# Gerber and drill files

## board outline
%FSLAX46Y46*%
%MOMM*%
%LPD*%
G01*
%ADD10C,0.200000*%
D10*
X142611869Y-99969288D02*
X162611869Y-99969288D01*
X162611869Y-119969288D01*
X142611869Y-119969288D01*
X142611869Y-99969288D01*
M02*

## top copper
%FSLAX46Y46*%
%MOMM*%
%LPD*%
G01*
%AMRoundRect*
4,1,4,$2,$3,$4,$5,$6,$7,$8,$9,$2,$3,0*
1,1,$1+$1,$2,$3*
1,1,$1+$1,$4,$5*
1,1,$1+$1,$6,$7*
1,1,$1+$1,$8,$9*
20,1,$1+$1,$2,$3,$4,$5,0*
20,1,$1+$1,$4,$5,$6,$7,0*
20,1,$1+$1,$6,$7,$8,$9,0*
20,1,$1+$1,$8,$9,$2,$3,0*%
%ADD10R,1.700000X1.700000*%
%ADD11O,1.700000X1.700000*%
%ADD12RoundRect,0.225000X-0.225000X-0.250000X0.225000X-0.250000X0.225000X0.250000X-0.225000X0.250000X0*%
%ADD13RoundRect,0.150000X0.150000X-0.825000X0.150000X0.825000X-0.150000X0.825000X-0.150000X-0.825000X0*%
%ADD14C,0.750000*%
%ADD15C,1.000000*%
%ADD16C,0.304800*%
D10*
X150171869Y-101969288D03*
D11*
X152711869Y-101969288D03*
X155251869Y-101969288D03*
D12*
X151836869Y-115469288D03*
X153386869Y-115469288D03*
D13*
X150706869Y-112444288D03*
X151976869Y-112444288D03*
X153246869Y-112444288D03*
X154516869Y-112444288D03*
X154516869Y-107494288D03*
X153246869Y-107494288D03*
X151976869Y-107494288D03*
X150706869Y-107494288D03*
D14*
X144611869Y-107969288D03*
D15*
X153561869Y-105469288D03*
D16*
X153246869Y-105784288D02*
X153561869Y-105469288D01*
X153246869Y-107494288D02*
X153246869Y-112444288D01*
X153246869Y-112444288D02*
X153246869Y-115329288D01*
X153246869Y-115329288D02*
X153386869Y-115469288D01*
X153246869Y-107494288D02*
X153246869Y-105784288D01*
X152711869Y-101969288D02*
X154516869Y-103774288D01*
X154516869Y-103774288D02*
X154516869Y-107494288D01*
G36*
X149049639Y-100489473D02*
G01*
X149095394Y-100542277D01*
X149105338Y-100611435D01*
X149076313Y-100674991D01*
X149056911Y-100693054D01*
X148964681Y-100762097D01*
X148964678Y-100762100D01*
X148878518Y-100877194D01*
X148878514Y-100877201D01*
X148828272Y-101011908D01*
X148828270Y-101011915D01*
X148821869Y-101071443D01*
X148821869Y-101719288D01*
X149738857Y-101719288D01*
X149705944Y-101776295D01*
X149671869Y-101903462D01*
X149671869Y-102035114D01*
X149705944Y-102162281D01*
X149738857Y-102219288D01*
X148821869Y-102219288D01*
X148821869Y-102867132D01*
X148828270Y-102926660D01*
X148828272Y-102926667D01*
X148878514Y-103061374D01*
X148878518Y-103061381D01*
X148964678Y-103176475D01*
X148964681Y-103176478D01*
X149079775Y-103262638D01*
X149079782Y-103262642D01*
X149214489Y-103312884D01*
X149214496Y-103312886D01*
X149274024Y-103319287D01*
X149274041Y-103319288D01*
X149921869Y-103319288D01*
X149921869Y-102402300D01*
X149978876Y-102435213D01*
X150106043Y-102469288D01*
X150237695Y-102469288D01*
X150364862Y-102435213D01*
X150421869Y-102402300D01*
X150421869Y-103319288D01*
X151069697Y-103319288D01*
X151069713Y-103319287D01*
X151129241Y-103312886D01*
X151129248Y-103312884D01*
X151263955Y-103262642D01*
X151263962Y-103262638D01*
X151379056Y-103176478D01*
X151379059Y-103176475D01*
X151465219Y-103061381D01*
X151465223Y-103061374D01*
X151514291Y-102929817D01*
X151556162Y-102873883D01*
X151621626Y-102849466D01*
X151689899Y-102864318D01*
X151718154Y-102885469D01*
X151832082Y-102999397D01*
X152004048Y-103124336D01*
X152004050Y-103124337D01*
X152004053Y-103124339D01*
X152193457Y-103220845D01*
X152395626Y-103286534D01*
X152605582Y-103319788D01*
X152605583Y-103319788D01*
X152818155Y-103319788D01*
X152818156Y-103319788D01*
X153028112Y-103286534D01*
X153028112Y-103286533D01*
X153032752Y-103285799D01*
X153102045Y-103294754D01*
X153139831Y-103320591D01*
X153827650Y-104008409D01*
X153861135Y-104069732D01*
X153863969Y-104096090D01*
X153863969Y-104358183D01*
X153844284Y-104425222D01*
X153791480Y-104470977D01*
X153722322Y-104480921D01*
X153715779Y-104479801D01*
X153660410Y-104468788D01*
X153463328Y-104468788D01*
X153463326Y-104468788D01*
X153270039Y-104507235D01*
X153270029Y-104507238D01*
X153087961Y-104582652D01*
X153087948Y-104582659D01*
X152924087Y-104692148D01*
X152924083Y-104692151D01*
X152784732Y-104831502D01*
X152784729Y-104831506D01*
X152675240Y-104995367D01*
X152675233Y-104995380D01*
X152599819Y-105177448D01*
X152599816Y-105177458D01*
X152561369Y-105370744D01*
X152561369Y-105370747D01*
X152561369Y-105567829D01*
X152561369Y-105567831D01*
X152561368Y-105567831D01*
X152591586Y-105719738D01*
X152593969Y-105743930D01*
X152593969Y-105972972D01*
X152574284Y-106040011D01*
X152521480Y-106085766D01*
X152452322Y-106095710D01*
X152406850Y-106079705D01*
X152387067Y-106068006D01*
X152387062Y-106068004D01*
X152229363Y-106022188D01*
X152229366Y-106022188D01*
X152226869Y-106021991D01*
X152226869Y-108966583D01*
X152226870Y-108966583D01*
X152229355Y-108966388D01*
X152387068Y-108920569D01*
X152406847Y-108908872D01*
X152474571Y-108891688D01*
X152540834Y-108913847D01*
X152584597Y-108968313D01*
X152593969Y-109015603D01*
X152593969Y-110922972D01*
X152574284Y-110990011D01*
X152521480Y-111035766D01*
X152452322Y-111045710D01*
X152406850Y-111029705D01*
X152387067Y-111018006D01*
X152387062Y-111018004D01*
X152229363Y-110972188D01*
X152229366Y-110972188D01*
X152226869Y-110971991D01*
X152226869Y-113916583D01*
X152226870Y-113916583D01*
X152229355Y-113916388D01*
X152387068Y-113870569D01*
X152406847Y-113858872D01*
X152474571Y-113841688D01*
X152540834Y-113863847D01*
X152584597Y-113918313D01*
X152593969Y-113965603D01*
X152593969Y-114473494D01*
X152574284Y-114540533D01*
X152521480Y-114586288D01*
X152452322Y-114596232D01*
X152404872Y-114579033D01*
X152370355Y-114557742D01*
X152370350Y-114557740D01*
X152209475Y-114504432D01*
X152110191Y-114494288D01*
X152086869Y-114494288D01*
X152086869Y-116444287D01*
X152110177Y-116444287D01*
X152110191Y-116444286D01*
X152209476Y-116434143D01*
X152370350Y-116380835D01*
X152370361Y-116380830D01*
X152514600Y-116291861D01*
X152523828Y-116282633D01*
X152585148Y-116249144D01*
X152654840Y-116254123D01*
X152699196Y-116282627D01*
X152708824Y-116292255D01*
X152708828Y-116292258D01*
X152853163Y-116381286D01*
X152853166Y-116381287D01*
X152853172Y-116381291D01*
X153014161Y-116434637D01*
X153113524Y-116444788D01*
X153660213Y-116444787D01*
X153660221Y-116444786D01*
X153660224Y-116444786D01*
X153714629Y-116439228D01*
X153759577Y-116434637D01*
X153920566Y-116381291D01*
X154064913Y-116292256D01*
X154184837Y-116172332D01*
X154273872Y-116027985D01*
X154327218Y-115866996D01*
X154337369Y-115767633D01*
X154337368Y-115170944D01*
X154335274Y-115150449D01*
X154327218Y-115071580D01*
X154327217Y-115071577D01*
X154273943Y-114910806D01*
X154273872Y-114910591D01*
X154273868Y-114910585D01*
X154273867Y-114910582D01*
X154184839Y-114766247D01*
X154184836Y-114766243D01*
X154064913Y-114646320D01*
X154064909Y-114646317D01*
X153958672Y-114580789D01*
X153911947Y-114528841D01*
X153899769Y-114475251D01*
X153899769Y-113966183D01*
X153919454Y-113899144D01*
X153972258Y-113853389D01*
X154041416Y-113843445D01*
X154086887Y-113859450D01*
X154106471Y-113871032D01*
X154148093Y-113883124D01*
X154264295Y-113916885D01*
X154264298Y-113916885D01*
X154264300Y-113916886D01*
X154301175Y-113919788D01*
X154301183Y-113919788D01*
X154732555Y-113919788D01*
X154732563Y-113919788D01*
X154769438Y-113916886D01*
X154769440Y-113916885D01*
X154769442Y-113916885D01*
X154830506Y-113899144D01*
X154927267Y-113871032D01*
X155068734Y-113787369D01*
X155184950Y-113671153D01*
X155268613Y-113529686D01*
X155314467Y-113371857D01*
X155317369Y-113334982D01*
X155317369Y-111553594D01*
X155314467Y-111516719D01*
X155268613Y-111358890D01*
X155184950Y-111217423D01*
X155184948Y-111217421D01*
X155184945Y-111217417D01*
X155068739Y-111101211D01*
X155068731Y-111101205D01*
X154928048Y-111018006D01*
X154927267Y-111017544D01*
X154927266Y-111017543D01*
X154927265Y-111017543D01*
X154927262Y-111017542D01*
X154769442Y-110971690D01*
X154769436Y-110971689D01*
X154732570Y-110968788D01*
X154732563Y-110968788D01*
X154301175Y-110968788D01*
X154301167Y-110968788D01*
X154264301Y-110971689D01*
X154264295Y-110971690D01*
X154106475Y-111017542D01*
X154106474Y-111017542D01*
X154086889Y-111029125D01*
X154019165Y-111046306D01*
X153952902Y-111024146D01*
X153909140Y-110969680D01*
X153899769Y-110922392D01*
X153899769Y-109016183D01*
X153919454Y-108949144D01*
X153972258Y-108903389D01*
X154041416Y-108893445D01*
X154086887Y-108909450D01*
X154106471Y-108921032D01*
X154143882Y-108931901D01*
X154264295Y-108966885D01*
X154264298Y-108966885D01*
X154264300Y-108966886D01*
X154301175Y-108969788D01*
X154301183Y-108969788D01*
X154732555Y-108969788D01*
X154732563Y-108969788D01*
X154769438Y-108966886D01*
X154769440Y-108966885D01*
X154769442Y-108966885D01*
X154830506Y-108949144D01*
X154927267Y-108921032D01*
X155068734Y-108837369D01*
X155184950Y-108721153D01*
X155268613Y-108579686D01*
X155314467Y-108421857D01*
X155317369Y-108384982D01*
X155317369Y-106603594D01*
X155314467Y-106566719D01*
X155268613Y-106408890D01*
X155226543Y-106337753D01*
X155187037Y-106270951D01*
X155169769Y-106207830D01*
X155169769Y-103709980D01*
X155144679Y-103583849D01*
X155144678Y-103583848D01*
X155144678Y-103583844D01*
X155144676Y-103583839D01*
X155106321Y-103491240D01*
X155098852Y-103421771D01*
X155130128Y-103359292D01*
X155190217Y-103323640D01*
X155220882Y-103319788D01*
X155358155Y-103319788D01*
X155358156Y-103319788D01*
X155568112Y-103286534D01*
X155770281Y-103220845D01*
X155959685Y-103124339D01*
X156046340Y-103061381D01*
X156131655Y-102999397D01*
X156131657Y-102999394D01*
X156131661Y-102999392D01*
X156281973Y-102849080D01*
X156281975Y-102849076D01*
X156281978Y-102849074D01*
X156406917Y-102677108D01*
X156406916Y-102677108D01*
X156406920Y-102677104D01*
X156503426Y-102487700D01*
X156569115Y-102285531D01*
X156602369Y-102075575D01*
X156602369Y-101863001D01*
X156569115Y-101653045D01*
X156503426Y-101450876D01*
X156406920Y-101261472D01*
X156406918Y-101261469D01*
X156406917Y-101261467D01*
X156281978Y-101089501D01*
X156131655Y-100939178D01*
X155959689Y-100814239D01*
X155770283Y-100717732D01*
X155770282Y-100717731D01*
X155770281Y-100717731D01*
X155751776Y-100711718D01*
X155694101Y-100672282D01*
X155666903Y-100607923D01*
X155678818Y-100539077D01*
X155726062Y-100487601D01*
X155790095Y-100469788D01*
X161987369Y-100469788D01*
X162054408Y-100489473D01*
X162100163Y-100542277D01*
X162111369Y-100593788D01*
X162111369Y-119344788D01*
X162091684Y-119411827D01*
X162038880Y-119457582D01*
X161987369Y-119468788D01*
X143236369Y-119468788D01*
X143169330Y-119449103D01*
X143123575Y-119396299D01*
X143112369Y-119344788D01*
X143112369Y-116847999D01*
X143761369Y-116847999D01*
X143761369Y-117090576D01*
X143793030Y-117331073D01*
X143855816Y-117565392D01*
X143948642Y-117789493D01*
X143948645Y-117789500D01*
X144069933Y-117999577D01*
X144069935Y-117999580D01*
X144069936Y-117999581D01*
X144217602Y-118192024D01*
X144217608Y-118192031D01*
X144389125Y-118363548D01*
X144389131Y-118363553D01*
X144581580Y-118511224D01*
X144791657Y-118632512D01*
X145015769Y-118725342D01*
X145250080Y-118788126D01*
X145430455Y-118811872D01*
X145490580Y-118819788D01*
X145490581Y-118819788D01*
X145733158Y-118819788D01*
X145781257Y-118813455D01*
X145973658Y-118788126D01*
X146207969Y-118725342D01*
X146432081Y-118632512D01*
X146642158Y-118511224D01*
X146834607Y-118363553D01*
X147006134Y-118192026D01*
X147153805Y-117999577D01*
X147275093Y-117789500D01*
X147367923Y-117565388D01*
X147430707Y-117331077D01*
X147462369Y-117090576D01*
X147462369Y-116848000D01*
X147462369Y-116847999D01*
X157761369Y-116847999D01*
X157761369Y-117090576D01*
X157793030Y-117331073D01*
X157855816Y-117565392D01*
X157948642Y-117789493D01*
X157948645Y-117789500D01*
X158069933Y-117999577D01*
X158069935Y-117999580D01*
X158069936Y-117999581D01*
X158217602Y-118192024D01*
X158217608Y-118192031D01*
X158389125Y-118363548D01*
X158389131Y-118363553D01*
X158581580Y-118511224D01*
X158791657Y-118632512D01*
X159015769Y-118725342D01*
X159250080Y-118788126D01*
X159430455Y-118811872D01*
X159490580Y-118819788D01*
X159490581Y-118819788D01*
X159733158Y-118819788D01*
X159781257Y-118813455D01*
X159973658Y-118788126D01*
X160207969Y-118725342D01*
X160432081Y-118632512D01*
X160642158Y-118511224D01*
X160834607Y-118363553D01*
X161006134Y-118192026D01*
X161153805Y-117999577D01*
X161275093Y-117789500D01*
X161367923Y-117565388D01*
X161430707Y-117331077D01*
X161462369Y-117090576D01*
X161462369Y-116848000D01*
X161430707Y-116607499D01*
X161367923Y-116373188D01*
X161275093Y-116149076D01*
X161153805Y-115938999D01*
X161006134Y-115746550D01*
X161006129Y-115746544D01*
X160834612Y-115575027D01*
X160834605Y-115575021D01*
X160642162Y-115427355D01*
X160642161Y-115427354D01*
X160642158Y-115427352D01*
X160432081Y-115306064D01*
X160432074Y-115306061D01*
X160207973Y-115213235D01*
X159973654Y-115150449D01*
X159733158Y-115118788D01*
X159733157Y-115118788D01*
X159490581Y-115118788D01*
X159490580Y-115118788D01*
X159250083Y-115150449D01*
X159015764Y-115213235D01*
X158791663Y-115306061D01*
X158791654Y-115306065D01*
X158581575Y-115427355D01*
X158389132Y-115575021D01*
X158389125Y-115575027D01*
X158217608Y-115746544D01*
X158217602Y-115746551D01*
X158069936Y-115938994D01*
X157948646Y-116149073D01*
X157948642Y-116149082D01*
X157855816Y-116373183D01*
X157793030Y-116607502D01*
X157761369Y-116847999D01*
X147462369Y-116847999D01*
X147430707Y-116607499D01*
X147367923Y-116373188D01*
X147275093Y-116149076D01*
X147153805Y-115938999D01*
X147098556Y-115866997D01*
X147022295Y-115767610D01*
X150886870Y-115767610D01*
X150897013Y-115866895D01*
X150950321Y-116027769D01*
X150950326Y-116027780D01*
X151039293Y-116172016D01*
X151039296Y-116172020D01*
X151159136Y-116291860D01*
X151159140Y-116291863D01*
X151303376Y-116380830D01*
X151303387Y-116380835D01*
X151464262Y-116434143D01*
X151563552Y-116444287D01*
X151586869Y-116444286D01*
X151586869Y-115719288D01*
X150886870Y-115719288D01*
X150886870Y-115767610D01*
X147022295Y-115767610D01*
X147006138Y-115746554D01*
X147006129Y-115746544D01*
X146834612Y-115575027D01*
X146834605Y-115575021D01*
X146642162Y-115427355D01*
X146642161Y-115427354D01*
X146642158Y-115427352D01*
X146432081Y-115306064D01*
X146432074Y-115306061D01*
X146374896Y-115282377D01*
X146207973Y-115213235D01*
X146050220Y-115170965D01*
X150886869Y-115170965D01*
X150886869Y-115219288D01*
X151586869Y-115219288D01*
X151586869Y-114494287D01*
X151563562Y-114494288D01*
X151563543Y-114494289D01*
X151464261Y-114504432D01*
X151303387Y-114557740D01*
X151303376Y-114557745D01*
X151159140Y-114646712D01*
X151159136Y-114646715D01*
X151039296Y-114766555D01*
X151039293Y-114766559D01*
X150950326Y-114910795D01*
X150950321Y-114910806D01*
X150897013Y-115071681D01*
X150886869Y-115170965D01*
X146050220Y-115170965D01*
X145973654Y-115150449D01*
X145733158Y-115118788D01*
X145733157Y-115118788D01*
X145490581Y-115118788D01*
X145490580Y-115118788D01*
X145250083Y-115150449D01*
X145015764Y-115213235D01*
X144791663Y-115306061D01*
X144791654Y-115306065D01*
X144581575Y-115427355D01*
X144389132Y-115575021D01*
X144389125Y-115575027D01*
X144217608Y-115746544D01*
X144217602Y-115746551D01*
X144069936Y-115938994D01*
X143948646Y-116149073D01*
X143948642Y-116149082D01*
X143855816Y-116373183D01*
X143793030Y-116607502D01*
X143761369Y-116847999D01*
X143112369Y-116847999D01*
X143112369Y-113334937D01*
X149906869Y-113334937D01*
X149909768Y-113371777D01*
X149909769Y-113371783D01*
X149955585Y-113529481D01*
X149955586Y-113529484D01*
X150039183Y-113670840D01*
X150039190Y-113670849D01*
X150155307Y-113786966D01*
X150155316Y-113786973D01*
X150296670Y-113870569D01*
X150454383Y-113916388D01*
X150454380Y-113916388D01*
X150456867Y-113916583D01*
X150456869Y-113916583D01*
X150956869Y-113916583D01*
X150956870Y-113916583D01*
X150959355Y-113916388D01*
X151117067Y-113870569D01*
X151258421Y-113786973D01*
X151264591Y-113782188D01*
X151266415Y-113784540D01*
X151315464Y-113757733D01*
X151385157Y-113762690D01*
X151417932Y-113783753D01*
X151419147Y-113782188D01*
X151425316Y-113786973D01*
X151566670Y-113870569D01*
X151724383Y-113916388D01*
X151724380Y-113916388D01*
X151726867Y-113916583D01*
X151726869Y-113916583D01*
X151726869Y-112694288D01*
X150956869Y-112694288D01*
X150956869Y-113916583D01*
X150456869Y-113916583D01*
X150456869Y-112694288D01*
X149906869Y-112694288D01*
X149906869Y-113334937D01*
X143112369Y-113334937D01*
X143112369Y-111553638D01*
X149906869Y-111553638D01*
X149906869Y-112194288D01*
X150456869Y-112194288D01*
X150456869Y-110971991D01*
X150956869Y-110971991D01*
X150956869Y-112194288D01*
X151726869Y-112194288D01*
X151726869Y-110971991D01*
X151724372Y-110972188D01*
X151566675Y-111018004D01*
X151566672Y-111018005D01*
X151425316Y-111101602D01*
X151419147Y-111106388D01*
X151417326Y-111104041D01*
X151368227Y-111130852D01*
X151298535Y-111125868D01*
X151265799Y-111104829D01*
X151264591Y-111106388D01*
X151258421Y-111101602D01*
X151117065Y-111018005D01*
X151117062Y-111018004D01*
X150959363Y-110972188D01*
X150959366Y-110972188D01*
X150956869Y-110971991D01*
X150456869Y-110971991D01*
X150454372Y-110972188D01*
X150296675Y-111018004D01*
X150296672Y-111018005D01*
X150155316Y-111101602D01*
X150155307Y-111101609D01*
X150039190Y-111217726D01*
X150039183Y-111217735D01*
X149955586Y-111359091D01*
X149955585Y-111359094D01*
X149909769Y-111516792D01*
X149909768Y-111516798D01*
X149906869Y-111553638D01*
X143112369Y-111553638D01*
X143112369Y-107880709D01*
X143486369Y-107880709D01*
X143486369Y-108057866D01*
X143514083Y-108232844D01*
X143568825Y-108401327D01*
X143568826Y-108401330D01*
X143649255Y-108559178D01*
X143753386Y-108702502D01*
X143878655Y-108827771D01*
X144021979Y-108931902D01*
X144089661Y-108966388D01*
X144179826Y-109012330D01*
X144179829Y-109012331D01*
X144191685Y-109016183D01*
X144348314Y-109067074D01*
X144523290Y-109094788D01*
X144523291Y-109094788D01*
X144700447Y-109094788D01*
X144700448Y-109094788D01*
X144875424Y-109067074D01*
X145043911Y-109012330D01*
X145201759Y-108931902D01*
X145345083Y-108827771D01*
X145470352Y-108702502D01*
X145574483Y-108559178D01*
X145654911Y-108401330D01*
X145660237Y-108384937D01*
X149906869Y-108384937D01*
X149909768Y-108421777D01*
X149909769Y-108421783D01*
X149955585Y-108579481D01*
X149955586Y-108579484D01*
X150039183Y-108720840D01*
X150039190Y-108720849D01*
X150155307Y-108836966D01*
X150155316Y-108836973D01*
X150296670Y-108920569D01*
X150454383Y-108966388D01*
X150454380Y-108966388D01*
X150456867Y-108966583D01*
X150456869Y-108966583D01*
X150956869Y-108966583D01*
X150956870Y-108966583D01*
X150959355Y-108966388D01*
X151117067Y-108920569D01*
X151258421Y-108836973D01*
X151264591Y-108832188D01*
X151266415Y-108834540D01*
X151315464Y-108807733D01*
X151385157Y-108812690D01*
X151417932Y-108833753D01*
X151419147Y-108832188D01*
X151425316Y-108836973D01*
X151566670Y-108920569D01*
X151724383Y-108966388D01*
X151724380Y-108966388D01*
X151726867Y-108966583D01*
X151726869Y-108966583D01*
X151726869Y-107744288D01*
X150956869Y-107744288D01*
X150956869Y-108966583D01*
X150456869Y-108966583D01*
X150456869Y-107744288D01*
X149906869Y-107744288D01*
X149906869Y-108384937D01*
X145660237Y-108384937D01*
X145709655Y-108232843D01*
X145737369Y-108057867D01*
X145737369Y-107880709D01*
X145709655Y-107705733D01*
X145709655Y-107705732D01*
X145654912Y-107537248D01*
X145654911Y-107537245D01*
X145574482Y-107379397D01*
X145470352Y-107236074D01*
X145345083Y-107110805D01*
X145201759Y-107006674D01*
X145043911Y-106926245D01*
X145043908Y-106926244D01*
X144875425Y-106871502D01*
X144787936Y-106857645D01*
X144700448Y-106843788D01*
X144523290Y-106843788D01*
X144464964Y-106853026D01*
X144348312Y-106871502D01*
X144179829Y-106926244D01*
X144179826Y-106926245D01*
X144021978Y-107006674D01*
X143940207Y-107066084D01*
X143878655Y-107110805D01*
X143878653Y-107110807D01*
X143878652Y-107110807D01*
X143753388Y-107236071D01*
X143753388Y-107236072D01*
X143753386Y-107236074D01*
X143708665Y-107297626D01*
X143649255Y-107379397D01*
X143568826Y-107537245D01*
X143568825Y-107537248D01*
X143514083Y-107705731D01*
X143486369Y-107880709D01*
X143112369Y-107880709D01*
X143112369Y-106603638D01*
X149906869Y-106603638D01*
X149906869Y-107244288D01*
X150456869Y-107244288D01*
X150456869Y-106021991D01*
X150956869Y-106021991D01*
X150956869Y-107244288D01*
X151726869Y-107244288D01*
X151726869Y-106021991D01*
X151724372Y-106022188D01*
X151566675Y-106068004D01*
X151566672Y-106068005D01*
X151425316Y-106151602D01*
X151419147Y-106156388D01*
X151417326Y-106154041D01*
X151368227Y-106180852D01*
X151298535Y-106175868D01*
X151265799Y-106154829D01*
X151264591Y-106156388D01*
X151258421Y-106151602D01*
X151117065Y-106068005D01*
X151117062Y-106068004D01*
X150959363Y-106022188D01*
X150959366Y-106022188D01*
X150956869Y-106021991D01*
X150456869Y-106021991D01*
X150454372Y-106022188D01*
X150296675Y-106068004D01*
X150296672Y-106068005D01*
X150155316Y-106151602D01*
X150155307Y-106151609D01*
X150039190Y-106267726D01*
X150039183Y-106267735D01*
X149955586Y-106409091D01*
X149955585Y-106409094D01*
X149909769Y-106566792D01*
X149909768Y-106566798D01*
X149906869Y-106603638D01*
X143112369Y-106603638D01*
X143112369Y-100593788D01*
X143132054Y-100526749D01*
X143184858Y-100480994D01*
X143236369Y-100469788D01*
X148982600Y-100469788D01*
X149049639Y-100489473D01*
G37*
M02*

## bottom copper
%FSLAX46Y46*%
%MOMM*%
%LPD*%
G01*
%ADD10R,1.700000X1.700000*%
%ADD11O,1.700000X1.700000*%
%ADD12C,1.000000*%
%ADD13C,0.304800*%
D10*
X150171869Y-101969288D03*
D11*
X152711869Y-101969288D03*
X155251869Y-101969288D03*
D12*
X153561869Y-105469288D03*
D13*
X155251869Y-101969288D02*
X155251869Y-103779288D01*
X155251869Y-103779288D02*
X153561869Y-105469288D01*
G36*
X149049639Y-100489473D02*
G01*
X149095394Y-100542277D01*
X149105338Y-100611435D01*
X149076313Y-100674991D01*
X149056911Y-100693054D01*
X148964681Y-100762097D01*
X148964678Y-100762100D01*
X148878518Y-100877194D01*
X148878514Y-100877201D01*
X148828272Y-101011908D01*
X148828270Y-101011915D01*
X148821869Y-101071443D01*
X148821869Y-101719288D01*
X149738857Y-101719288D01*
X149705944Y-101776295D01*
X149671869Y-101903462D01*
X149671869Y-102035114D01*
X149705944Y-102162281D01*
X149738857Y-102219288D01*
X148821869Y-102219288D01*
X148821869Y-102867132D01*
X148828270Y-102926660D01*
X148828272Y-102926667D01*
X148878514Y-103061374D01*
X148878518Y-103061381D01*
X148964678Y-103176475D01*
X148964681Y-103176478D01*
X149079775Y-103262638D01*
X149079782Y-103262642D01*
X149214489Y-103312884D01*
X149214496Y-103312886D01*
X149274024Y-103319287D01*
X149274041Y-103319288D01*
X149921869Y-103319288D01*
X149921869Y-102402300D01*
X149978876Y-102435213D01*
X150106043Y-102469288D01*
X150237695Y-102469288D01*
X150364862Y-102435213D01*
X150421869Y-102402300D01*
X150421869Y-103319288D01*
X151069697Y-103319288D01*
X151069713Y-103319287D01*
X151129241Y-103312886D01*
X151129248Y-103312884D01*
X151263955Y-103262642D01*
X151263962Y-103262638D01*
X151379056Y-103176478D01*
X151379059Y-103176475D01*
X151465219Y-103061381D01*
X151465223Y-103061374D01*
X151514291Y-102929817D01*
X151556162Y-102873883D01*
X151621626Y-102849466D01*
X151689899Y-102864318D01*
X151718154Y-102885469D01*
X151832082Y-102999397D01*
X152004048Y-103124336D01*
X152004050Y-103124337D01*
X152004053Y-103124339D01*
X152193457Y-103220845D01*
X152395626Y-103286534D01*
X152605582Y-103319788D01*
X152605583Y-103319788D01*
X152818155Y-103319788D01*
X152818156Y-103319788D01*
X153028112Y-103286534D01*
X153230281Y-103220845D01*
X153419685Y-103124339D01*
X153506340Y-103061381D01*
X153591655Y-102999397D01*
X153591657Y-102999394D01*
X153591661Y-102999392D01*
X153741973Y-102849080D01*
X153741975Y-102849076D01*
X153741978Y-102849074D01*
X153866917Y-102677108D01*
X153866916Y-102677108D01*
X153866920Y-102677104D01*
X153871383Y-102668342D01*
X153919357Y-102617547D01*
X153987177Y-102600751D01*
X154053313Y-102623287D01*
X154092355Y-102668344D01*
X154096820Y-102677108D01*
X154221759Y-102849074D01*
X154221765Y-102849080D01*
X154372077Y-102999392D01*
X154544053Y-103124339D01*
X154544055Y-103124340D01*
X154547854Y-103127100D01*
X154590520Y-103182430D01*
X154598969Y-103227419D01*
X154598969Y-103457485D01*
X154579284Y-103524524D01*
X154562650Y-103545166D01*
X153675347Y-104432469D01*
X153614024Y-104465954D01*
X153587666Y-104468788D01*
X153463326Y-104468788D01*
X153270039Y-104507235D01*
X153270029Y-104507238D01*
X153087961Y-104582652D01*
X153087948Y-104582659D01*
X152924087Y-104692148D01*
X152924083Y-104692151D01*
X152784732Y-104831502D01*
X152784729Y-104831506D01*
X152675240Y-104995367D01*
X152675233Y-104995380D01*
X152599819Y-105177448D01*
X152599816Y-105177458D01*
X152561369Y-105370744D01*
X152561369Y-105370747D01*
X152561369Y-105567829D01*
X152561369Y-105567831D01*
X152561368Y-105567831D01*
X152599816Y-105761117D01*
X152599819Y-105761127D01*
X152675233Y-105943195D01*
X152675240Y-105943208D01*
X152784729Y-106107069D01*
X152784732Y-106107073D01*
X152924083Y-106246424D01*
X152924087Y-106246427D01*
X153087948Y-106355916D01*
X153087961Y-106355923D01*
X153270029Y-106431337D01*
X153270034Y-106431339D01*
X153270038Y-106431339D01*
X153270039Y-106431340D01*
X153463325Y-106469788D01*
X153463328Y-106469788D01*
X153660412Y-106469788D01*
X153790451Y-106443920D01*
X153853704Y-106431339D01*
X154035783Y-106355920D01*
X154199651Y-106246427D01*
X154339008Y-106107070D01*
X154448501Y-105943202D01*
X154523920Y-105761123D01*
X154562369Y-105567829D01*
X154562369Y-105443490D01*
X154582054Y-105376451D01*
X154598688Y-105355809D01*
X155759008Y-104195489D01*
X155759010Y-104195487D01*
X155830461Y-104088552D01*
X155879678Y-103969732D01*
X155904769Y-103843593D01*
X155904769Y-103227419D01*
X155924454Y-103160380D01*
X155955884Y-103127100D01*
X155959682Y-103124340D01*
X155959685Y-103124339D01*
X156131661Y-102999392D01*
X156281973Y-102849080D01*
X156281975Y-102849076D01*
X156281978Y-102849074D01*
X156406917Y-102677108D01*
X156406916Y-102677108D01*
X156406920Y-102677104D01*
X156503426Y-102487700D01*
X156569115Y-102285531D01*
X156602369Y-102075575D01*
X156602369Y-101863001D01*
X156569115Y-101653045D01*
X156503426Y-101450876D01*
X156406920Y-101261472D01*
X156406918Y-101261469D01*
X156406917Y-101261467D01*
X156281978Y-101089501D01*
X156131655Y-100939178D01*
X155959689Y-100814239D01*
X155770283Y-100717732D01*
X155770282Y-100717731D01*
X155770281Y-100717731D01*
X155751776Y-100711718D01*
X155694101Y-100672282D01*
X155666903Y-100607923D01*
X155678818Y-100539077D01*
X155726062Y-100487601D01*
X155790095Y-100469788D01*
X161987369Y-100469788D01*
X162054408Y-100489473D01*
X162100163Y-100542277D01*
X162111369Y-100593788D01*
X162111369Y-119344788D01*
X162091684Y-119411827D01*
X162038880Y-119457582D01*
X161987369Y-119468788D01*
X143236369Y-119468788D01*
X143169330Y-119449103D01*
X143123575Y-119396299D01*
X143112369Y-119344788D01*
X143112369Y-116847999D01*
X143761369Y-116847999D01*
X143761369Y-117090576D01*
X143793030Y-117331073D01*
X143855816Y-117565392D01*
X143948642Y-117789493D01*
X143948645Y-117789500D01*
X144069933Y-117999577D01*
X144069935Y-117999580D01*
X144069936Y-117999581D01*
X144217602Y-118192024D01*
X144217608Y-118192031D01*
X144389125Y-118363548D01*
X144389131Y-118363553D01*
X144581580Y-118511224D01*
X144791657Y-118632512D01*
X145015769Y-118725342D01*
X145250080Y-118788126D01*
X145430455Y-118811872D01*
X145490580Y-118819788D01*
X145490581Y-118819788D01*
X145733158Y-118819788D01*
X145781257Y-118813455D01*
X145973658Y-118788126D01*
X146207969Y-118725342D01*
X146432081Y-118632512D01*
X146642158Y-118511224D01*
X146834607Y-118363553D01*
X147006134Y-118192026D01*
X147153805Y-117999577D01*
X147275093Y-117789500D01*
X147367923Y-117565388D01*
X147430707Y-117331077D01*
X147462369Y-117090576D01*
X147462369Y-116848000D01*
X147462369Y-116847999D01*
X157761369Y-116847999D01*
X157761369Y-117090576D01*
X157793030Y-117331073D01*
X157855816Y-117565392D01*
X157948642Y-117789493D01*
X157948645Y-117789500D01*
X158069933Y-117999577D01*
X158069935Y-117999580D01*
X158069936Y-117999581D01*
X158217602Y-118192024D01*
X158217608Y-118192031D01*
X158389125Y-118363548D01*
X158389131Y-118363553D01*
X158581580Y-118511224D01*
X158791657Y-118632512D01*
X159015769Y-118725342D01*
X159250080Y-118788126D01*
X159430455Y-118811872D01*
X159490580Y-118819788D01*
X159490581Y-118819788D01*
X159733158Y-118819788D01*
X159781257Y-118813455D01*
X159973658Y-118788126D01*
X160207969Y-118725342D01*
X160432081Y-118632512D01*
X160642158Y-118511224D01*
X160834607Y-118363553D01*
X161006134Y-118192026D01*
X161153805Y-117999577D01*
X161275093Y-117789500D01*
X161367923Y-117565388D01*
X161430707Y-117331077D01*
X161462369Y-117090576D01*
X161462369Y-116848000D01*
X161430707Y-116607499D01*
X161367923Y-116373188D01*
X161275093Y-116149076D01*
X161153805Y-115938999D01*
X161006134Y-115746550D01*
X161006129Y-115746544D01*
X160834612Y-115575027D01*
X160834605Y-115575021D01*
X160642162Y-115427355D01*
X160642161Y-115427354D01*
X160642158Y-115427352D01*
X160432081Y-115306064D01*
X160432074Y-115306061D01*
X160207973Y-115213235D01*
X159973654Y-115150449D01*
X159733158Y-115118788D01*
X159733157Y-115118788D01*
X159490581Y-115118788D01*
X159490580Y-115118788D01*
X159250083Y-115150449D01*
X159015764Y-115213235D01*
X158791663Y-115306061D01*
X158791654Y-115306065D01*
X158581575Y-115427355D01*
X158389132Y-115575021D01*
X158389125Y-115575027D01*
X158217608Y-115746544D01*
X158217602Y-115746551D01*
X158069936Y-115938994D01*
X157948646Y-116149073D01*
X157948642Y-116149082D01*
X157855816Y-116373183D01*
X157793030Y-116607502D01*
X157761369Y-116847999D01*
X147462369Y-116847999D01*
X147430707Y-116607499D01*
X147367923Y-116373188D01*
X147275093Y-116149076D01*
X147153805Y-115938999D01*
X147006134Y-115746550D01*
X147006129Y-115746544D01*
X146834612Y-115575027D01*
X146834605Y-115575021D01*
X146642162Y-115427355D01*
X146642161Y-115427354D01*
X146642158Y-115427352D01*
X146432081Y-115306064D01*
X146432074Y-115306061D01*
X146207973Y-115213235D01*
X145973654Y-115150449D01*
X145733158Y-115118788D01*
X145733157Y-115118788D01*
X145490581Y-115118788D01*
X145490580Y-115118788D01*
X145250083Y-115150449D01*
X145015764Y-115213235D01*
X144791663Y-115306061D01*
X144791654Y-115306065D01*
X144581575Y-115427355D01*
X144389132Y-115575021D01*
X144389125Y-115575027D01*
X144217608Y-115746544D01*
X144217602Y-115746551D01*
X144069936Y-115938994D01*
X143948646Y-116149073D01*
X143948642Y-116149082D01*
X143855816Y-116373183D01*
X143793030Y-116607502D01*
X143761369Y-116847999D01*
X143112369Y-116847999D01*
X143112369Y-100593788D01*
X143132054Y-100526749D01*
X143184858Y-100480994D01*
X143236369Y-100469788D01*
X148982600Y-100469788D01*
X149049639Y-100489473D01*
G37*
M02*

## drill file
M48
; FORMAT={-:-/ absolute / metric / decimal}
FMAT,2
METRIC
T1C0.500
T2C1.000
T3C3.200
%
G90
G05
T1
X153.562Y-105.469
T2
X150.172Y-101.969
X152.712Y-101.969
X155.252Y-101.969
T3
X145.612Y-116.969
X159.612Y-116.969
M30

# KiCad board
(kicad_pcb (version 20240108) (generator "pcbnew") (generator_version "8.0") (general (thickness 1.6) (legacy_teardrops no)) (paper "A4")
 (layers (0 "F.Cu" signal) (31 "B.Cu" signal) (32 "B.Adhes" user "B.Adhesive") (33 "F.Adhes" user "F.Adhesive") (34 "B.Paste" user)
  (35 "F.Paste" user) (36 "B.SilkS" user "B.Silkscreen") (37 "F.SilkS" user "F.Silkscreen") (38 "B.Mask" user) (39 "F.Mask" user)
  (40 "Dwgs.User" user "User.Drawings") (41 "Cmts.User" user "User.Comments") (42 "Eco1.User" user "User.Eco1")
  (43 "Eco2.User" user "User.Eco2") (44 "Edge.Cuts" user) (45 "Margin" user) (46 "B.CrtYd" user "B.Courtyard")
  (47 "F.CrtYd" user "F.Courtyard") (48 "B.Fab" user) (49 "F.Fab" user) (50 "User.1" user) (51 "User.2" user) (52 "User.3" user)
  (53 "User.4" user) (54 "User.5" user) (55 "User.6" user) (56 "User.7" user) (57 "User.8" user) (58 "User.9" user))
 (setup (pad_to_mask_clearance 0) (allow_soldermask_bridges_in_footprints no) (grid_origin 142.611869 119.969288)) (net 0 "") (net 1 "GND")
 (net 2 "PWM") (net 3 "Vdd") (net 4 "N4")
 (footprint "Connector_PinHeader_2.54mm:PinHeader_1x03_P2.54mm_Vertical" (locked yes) (layer "F.Cu") (at 150.171869 101.969288 90)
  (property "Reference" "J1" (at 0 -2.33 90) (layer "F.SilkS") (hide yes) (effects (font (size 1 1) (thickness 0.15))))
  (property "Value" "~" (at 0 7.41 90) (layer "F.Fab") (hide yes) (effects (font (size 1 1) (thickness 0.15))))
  (pad "1" thru_hole rect (at 0 0 90) (size 1.7 1.7) (drill 1) (layers "*.Cu" "*.Mask") (remove_unused_layers no) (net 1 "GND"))
  (pad "2" thru_hole oval (at 0 2.54 90) (size 1.7 1.7) (drill 1) (layers "*.Cu" "*.Mask") (remove_unused_layers no) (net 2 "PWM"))
  (pad "3" thru_hole oval (at 0 5.08 90) (size 1.7 1.7) (drill 1) (layers "*.Cu" "*.Mask") (remove_unused_layers no) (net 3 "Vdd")))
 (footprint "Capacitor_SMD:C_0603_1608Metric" (layer "F.Cu") (at 152.611869 115.469288)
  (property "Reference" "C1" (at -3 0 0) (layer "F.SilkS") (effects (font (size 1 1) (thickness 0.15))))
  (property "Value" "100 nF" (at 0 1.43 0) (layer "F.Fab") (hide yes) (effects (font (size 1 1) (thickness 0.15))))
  (pad "1" smd roundrect (at -0.775 0) (size 0.9 0.95) (layers "F.Cu" "F.Paste" "F.Mask") (roundrect_rratio 0.25) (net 1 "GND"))
  (pad "2" smd roundrect (at 0.775 0) (size 0.9 0.95) (layers "F.Cu" "F.Paste" "F.Mask") (roundrect_rratio 0.25) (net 3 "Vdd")))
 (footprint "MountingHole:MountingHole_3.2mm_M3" (layer "F.Cu") (at 159.611869 116.969288)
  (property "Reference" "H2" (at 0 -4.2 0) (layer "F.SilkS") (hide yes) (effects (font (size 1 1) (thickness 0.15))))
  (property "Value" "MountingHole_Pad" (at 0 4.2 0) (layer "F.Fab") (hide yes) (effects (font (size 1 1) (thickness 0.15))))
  (pad "" np_thru_hole circle (at 0 0) (size 3.2 3.2) (drill 3.2) (layers "*.Cu" "*.Mask")))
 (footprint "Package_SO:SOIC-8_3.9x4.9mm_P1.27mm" (layer "F.Cu") (at 152.611869 109.969288 90)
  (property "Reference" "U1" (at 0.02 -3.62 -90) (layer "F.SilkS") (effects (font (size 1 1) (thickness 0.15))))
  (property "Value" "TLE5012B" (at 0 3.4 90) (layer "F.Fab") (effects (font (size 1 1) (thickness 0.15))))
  (pad "1" smd roundrect (at -2.475 -1.905 90) (size 1.95 0.6) (layers "F.Cu" "F.Paste" "F.Mask") (roundrect_rratio 0.25) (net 1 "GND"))
  (pad "2" smd roundrect (at -2.475 -0.635 90) (size 1.95 0.6) (layers "F.Cu" "F.Paste" "F.Mask") (roundrect_rratio 0.25) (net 1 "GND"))
  (pad "3" smd roundrect (at -2.475 0.635 90) (size 1.95 0.6) (layers "F.Cu" "F.Paste" "F.Mask") (roundrect_rratio 0.25) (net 3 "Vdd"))
  (pad "4" smd roundrect (at -2.475 1.905 90) (size 1.95 0.6) (layers "F.Cu" "F.Paste" "F.Mask") (roundrect_rratio 0.25) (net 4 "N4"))
  (pad "5" smd roundrect (at 2.475 1.905 90) (size 1.95 0.6) (layers "F.Cu" "F.Paste" "F.Mask") (roundrect_rratio 0.25) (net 2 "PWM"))
  (pad "6" smd roundrect (at 2.475 0.635 90) (size 1.95 0.6) (layers "F.Cu" "F.Paste" "F.Mask") (roundrect_rratio 0.25) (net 3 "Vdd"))
  (pad "7" smd roundrect (at 2.475 -0.635 90) (size 1.95 0.6) (layers "F.Cu" "F.Paste" "F.Mask") (roundrect_rratio 0.25) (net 1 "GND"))
  (pad "8" smd roundrect (at 2.475 -1.905 90) (size 1.95 0.6) (layers "F.Cu" "F.Paste" "F.Mask") (roundrect_rratio 0.25) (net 1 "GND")))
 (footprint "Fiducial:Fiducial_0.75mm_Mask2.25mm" (layer "F.Cu") (at 144.611869 107.969288)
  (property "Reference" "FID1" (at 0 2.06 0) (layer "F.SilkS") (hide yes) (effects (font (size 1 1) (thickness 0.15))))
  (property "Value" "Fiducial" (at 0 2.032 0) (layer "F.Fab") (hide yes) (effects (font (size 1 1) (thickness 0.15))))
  (pad "" smd circle (at 0 0) (size 0.75 0.75) (layers "F.Cu" "F.Mask") (solder_mask_margin 0.75) (clearance 0.75)))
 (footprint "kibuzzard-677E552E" (layer "F.Cu") (at 150.171869 104.616321 90)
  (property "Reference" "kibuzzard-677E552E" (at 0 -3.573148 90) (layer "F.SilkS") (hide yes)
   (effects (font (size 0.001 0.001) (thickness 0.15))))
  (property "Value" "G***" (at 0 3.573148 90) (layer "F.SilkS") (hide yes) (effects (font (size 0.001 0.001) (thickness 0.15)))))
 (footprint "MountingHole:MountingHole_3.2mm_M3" (layer "F.Cu") (at 145.611869 116.969288)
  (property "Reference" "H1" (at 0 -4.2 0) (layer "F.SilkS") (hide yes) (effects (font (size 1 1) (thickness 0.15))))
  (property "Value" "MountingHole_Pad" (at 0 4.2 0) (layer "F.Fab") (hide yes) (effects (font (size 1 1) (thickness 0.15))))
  (pad "" np_thru_hole circle (at 0 0) (size 3.2 3.2) (drill 3.2) (layers "*.Cu" "*.Mask")))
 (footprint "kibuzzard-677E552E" (layer "B.Cu") (at 150.171869 104.283306 -90)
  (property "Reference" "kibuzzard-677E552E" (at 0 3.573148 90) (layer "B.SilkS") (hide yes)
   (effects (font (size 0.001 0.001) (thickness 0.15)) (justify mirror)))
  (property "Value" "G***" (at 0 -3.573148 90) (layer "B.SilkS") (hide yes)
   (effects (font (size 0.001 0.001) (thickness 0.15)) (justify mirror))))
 (gr_rect (start 142.611869 99.969288) (end 162.611869 119.969288) (stroke (width 0.2) (type default)) (fill none) (layer "Edge.Cuts"))
 (segment (start 153.246869 105.784288) (end 153.561869 105.469288) (width 0.3048) (layer "F.Cu") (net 3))
 (segment (start 153.246869 107.494288) (end 153.246869 112.444288) (width 0.3048) (layer "F.Cu") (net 3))
 (segment (start 153.246869 112.444288) (end 153.246869 115.329288) (width 0.3048) (layer "F.Cu") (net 3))
 (segment (start 153.246869 115.329288) (end 153.386869 115.469288) (width 0.3048) (layer "F.Cu") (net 3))
 (segment (start 153.246869 107.494288) (end 153.246869 105.784288) (width 0.3048) (layer "F.Cu") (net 3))
 (via (at 153.561869 105.469288) (size 1) (drill 0.5) (layers "F.Cu" "B.Cu") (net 3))
 (segment (start 155.251869 101.969288) (end 155.251869 103.779288) (width 0.3048) (layer "B.Cu") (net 3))
 (segment (start 155.251869 103.779288) (end 153.561869 105.469288) (width 0.3048) (layer "B.Cu") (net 3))
 (segment (start 152.711869 101.969288) (end 154.516869 103.774288) (width 0.3048) (layer "F.Cu") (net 2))
 (segment (start 154.516869 103.774288) (end 154.516869 107.494288) (width 0.3048) (layer "F.Cu") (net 2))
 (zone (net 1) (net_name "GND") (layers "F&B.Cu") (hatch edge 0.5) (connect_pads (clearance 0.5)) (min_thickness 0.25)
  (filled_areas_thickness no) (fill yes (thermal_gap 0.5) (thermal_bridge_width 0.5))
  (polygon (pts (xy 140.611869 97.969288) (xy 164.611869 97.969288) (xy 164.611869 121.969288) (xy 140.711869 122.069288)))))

